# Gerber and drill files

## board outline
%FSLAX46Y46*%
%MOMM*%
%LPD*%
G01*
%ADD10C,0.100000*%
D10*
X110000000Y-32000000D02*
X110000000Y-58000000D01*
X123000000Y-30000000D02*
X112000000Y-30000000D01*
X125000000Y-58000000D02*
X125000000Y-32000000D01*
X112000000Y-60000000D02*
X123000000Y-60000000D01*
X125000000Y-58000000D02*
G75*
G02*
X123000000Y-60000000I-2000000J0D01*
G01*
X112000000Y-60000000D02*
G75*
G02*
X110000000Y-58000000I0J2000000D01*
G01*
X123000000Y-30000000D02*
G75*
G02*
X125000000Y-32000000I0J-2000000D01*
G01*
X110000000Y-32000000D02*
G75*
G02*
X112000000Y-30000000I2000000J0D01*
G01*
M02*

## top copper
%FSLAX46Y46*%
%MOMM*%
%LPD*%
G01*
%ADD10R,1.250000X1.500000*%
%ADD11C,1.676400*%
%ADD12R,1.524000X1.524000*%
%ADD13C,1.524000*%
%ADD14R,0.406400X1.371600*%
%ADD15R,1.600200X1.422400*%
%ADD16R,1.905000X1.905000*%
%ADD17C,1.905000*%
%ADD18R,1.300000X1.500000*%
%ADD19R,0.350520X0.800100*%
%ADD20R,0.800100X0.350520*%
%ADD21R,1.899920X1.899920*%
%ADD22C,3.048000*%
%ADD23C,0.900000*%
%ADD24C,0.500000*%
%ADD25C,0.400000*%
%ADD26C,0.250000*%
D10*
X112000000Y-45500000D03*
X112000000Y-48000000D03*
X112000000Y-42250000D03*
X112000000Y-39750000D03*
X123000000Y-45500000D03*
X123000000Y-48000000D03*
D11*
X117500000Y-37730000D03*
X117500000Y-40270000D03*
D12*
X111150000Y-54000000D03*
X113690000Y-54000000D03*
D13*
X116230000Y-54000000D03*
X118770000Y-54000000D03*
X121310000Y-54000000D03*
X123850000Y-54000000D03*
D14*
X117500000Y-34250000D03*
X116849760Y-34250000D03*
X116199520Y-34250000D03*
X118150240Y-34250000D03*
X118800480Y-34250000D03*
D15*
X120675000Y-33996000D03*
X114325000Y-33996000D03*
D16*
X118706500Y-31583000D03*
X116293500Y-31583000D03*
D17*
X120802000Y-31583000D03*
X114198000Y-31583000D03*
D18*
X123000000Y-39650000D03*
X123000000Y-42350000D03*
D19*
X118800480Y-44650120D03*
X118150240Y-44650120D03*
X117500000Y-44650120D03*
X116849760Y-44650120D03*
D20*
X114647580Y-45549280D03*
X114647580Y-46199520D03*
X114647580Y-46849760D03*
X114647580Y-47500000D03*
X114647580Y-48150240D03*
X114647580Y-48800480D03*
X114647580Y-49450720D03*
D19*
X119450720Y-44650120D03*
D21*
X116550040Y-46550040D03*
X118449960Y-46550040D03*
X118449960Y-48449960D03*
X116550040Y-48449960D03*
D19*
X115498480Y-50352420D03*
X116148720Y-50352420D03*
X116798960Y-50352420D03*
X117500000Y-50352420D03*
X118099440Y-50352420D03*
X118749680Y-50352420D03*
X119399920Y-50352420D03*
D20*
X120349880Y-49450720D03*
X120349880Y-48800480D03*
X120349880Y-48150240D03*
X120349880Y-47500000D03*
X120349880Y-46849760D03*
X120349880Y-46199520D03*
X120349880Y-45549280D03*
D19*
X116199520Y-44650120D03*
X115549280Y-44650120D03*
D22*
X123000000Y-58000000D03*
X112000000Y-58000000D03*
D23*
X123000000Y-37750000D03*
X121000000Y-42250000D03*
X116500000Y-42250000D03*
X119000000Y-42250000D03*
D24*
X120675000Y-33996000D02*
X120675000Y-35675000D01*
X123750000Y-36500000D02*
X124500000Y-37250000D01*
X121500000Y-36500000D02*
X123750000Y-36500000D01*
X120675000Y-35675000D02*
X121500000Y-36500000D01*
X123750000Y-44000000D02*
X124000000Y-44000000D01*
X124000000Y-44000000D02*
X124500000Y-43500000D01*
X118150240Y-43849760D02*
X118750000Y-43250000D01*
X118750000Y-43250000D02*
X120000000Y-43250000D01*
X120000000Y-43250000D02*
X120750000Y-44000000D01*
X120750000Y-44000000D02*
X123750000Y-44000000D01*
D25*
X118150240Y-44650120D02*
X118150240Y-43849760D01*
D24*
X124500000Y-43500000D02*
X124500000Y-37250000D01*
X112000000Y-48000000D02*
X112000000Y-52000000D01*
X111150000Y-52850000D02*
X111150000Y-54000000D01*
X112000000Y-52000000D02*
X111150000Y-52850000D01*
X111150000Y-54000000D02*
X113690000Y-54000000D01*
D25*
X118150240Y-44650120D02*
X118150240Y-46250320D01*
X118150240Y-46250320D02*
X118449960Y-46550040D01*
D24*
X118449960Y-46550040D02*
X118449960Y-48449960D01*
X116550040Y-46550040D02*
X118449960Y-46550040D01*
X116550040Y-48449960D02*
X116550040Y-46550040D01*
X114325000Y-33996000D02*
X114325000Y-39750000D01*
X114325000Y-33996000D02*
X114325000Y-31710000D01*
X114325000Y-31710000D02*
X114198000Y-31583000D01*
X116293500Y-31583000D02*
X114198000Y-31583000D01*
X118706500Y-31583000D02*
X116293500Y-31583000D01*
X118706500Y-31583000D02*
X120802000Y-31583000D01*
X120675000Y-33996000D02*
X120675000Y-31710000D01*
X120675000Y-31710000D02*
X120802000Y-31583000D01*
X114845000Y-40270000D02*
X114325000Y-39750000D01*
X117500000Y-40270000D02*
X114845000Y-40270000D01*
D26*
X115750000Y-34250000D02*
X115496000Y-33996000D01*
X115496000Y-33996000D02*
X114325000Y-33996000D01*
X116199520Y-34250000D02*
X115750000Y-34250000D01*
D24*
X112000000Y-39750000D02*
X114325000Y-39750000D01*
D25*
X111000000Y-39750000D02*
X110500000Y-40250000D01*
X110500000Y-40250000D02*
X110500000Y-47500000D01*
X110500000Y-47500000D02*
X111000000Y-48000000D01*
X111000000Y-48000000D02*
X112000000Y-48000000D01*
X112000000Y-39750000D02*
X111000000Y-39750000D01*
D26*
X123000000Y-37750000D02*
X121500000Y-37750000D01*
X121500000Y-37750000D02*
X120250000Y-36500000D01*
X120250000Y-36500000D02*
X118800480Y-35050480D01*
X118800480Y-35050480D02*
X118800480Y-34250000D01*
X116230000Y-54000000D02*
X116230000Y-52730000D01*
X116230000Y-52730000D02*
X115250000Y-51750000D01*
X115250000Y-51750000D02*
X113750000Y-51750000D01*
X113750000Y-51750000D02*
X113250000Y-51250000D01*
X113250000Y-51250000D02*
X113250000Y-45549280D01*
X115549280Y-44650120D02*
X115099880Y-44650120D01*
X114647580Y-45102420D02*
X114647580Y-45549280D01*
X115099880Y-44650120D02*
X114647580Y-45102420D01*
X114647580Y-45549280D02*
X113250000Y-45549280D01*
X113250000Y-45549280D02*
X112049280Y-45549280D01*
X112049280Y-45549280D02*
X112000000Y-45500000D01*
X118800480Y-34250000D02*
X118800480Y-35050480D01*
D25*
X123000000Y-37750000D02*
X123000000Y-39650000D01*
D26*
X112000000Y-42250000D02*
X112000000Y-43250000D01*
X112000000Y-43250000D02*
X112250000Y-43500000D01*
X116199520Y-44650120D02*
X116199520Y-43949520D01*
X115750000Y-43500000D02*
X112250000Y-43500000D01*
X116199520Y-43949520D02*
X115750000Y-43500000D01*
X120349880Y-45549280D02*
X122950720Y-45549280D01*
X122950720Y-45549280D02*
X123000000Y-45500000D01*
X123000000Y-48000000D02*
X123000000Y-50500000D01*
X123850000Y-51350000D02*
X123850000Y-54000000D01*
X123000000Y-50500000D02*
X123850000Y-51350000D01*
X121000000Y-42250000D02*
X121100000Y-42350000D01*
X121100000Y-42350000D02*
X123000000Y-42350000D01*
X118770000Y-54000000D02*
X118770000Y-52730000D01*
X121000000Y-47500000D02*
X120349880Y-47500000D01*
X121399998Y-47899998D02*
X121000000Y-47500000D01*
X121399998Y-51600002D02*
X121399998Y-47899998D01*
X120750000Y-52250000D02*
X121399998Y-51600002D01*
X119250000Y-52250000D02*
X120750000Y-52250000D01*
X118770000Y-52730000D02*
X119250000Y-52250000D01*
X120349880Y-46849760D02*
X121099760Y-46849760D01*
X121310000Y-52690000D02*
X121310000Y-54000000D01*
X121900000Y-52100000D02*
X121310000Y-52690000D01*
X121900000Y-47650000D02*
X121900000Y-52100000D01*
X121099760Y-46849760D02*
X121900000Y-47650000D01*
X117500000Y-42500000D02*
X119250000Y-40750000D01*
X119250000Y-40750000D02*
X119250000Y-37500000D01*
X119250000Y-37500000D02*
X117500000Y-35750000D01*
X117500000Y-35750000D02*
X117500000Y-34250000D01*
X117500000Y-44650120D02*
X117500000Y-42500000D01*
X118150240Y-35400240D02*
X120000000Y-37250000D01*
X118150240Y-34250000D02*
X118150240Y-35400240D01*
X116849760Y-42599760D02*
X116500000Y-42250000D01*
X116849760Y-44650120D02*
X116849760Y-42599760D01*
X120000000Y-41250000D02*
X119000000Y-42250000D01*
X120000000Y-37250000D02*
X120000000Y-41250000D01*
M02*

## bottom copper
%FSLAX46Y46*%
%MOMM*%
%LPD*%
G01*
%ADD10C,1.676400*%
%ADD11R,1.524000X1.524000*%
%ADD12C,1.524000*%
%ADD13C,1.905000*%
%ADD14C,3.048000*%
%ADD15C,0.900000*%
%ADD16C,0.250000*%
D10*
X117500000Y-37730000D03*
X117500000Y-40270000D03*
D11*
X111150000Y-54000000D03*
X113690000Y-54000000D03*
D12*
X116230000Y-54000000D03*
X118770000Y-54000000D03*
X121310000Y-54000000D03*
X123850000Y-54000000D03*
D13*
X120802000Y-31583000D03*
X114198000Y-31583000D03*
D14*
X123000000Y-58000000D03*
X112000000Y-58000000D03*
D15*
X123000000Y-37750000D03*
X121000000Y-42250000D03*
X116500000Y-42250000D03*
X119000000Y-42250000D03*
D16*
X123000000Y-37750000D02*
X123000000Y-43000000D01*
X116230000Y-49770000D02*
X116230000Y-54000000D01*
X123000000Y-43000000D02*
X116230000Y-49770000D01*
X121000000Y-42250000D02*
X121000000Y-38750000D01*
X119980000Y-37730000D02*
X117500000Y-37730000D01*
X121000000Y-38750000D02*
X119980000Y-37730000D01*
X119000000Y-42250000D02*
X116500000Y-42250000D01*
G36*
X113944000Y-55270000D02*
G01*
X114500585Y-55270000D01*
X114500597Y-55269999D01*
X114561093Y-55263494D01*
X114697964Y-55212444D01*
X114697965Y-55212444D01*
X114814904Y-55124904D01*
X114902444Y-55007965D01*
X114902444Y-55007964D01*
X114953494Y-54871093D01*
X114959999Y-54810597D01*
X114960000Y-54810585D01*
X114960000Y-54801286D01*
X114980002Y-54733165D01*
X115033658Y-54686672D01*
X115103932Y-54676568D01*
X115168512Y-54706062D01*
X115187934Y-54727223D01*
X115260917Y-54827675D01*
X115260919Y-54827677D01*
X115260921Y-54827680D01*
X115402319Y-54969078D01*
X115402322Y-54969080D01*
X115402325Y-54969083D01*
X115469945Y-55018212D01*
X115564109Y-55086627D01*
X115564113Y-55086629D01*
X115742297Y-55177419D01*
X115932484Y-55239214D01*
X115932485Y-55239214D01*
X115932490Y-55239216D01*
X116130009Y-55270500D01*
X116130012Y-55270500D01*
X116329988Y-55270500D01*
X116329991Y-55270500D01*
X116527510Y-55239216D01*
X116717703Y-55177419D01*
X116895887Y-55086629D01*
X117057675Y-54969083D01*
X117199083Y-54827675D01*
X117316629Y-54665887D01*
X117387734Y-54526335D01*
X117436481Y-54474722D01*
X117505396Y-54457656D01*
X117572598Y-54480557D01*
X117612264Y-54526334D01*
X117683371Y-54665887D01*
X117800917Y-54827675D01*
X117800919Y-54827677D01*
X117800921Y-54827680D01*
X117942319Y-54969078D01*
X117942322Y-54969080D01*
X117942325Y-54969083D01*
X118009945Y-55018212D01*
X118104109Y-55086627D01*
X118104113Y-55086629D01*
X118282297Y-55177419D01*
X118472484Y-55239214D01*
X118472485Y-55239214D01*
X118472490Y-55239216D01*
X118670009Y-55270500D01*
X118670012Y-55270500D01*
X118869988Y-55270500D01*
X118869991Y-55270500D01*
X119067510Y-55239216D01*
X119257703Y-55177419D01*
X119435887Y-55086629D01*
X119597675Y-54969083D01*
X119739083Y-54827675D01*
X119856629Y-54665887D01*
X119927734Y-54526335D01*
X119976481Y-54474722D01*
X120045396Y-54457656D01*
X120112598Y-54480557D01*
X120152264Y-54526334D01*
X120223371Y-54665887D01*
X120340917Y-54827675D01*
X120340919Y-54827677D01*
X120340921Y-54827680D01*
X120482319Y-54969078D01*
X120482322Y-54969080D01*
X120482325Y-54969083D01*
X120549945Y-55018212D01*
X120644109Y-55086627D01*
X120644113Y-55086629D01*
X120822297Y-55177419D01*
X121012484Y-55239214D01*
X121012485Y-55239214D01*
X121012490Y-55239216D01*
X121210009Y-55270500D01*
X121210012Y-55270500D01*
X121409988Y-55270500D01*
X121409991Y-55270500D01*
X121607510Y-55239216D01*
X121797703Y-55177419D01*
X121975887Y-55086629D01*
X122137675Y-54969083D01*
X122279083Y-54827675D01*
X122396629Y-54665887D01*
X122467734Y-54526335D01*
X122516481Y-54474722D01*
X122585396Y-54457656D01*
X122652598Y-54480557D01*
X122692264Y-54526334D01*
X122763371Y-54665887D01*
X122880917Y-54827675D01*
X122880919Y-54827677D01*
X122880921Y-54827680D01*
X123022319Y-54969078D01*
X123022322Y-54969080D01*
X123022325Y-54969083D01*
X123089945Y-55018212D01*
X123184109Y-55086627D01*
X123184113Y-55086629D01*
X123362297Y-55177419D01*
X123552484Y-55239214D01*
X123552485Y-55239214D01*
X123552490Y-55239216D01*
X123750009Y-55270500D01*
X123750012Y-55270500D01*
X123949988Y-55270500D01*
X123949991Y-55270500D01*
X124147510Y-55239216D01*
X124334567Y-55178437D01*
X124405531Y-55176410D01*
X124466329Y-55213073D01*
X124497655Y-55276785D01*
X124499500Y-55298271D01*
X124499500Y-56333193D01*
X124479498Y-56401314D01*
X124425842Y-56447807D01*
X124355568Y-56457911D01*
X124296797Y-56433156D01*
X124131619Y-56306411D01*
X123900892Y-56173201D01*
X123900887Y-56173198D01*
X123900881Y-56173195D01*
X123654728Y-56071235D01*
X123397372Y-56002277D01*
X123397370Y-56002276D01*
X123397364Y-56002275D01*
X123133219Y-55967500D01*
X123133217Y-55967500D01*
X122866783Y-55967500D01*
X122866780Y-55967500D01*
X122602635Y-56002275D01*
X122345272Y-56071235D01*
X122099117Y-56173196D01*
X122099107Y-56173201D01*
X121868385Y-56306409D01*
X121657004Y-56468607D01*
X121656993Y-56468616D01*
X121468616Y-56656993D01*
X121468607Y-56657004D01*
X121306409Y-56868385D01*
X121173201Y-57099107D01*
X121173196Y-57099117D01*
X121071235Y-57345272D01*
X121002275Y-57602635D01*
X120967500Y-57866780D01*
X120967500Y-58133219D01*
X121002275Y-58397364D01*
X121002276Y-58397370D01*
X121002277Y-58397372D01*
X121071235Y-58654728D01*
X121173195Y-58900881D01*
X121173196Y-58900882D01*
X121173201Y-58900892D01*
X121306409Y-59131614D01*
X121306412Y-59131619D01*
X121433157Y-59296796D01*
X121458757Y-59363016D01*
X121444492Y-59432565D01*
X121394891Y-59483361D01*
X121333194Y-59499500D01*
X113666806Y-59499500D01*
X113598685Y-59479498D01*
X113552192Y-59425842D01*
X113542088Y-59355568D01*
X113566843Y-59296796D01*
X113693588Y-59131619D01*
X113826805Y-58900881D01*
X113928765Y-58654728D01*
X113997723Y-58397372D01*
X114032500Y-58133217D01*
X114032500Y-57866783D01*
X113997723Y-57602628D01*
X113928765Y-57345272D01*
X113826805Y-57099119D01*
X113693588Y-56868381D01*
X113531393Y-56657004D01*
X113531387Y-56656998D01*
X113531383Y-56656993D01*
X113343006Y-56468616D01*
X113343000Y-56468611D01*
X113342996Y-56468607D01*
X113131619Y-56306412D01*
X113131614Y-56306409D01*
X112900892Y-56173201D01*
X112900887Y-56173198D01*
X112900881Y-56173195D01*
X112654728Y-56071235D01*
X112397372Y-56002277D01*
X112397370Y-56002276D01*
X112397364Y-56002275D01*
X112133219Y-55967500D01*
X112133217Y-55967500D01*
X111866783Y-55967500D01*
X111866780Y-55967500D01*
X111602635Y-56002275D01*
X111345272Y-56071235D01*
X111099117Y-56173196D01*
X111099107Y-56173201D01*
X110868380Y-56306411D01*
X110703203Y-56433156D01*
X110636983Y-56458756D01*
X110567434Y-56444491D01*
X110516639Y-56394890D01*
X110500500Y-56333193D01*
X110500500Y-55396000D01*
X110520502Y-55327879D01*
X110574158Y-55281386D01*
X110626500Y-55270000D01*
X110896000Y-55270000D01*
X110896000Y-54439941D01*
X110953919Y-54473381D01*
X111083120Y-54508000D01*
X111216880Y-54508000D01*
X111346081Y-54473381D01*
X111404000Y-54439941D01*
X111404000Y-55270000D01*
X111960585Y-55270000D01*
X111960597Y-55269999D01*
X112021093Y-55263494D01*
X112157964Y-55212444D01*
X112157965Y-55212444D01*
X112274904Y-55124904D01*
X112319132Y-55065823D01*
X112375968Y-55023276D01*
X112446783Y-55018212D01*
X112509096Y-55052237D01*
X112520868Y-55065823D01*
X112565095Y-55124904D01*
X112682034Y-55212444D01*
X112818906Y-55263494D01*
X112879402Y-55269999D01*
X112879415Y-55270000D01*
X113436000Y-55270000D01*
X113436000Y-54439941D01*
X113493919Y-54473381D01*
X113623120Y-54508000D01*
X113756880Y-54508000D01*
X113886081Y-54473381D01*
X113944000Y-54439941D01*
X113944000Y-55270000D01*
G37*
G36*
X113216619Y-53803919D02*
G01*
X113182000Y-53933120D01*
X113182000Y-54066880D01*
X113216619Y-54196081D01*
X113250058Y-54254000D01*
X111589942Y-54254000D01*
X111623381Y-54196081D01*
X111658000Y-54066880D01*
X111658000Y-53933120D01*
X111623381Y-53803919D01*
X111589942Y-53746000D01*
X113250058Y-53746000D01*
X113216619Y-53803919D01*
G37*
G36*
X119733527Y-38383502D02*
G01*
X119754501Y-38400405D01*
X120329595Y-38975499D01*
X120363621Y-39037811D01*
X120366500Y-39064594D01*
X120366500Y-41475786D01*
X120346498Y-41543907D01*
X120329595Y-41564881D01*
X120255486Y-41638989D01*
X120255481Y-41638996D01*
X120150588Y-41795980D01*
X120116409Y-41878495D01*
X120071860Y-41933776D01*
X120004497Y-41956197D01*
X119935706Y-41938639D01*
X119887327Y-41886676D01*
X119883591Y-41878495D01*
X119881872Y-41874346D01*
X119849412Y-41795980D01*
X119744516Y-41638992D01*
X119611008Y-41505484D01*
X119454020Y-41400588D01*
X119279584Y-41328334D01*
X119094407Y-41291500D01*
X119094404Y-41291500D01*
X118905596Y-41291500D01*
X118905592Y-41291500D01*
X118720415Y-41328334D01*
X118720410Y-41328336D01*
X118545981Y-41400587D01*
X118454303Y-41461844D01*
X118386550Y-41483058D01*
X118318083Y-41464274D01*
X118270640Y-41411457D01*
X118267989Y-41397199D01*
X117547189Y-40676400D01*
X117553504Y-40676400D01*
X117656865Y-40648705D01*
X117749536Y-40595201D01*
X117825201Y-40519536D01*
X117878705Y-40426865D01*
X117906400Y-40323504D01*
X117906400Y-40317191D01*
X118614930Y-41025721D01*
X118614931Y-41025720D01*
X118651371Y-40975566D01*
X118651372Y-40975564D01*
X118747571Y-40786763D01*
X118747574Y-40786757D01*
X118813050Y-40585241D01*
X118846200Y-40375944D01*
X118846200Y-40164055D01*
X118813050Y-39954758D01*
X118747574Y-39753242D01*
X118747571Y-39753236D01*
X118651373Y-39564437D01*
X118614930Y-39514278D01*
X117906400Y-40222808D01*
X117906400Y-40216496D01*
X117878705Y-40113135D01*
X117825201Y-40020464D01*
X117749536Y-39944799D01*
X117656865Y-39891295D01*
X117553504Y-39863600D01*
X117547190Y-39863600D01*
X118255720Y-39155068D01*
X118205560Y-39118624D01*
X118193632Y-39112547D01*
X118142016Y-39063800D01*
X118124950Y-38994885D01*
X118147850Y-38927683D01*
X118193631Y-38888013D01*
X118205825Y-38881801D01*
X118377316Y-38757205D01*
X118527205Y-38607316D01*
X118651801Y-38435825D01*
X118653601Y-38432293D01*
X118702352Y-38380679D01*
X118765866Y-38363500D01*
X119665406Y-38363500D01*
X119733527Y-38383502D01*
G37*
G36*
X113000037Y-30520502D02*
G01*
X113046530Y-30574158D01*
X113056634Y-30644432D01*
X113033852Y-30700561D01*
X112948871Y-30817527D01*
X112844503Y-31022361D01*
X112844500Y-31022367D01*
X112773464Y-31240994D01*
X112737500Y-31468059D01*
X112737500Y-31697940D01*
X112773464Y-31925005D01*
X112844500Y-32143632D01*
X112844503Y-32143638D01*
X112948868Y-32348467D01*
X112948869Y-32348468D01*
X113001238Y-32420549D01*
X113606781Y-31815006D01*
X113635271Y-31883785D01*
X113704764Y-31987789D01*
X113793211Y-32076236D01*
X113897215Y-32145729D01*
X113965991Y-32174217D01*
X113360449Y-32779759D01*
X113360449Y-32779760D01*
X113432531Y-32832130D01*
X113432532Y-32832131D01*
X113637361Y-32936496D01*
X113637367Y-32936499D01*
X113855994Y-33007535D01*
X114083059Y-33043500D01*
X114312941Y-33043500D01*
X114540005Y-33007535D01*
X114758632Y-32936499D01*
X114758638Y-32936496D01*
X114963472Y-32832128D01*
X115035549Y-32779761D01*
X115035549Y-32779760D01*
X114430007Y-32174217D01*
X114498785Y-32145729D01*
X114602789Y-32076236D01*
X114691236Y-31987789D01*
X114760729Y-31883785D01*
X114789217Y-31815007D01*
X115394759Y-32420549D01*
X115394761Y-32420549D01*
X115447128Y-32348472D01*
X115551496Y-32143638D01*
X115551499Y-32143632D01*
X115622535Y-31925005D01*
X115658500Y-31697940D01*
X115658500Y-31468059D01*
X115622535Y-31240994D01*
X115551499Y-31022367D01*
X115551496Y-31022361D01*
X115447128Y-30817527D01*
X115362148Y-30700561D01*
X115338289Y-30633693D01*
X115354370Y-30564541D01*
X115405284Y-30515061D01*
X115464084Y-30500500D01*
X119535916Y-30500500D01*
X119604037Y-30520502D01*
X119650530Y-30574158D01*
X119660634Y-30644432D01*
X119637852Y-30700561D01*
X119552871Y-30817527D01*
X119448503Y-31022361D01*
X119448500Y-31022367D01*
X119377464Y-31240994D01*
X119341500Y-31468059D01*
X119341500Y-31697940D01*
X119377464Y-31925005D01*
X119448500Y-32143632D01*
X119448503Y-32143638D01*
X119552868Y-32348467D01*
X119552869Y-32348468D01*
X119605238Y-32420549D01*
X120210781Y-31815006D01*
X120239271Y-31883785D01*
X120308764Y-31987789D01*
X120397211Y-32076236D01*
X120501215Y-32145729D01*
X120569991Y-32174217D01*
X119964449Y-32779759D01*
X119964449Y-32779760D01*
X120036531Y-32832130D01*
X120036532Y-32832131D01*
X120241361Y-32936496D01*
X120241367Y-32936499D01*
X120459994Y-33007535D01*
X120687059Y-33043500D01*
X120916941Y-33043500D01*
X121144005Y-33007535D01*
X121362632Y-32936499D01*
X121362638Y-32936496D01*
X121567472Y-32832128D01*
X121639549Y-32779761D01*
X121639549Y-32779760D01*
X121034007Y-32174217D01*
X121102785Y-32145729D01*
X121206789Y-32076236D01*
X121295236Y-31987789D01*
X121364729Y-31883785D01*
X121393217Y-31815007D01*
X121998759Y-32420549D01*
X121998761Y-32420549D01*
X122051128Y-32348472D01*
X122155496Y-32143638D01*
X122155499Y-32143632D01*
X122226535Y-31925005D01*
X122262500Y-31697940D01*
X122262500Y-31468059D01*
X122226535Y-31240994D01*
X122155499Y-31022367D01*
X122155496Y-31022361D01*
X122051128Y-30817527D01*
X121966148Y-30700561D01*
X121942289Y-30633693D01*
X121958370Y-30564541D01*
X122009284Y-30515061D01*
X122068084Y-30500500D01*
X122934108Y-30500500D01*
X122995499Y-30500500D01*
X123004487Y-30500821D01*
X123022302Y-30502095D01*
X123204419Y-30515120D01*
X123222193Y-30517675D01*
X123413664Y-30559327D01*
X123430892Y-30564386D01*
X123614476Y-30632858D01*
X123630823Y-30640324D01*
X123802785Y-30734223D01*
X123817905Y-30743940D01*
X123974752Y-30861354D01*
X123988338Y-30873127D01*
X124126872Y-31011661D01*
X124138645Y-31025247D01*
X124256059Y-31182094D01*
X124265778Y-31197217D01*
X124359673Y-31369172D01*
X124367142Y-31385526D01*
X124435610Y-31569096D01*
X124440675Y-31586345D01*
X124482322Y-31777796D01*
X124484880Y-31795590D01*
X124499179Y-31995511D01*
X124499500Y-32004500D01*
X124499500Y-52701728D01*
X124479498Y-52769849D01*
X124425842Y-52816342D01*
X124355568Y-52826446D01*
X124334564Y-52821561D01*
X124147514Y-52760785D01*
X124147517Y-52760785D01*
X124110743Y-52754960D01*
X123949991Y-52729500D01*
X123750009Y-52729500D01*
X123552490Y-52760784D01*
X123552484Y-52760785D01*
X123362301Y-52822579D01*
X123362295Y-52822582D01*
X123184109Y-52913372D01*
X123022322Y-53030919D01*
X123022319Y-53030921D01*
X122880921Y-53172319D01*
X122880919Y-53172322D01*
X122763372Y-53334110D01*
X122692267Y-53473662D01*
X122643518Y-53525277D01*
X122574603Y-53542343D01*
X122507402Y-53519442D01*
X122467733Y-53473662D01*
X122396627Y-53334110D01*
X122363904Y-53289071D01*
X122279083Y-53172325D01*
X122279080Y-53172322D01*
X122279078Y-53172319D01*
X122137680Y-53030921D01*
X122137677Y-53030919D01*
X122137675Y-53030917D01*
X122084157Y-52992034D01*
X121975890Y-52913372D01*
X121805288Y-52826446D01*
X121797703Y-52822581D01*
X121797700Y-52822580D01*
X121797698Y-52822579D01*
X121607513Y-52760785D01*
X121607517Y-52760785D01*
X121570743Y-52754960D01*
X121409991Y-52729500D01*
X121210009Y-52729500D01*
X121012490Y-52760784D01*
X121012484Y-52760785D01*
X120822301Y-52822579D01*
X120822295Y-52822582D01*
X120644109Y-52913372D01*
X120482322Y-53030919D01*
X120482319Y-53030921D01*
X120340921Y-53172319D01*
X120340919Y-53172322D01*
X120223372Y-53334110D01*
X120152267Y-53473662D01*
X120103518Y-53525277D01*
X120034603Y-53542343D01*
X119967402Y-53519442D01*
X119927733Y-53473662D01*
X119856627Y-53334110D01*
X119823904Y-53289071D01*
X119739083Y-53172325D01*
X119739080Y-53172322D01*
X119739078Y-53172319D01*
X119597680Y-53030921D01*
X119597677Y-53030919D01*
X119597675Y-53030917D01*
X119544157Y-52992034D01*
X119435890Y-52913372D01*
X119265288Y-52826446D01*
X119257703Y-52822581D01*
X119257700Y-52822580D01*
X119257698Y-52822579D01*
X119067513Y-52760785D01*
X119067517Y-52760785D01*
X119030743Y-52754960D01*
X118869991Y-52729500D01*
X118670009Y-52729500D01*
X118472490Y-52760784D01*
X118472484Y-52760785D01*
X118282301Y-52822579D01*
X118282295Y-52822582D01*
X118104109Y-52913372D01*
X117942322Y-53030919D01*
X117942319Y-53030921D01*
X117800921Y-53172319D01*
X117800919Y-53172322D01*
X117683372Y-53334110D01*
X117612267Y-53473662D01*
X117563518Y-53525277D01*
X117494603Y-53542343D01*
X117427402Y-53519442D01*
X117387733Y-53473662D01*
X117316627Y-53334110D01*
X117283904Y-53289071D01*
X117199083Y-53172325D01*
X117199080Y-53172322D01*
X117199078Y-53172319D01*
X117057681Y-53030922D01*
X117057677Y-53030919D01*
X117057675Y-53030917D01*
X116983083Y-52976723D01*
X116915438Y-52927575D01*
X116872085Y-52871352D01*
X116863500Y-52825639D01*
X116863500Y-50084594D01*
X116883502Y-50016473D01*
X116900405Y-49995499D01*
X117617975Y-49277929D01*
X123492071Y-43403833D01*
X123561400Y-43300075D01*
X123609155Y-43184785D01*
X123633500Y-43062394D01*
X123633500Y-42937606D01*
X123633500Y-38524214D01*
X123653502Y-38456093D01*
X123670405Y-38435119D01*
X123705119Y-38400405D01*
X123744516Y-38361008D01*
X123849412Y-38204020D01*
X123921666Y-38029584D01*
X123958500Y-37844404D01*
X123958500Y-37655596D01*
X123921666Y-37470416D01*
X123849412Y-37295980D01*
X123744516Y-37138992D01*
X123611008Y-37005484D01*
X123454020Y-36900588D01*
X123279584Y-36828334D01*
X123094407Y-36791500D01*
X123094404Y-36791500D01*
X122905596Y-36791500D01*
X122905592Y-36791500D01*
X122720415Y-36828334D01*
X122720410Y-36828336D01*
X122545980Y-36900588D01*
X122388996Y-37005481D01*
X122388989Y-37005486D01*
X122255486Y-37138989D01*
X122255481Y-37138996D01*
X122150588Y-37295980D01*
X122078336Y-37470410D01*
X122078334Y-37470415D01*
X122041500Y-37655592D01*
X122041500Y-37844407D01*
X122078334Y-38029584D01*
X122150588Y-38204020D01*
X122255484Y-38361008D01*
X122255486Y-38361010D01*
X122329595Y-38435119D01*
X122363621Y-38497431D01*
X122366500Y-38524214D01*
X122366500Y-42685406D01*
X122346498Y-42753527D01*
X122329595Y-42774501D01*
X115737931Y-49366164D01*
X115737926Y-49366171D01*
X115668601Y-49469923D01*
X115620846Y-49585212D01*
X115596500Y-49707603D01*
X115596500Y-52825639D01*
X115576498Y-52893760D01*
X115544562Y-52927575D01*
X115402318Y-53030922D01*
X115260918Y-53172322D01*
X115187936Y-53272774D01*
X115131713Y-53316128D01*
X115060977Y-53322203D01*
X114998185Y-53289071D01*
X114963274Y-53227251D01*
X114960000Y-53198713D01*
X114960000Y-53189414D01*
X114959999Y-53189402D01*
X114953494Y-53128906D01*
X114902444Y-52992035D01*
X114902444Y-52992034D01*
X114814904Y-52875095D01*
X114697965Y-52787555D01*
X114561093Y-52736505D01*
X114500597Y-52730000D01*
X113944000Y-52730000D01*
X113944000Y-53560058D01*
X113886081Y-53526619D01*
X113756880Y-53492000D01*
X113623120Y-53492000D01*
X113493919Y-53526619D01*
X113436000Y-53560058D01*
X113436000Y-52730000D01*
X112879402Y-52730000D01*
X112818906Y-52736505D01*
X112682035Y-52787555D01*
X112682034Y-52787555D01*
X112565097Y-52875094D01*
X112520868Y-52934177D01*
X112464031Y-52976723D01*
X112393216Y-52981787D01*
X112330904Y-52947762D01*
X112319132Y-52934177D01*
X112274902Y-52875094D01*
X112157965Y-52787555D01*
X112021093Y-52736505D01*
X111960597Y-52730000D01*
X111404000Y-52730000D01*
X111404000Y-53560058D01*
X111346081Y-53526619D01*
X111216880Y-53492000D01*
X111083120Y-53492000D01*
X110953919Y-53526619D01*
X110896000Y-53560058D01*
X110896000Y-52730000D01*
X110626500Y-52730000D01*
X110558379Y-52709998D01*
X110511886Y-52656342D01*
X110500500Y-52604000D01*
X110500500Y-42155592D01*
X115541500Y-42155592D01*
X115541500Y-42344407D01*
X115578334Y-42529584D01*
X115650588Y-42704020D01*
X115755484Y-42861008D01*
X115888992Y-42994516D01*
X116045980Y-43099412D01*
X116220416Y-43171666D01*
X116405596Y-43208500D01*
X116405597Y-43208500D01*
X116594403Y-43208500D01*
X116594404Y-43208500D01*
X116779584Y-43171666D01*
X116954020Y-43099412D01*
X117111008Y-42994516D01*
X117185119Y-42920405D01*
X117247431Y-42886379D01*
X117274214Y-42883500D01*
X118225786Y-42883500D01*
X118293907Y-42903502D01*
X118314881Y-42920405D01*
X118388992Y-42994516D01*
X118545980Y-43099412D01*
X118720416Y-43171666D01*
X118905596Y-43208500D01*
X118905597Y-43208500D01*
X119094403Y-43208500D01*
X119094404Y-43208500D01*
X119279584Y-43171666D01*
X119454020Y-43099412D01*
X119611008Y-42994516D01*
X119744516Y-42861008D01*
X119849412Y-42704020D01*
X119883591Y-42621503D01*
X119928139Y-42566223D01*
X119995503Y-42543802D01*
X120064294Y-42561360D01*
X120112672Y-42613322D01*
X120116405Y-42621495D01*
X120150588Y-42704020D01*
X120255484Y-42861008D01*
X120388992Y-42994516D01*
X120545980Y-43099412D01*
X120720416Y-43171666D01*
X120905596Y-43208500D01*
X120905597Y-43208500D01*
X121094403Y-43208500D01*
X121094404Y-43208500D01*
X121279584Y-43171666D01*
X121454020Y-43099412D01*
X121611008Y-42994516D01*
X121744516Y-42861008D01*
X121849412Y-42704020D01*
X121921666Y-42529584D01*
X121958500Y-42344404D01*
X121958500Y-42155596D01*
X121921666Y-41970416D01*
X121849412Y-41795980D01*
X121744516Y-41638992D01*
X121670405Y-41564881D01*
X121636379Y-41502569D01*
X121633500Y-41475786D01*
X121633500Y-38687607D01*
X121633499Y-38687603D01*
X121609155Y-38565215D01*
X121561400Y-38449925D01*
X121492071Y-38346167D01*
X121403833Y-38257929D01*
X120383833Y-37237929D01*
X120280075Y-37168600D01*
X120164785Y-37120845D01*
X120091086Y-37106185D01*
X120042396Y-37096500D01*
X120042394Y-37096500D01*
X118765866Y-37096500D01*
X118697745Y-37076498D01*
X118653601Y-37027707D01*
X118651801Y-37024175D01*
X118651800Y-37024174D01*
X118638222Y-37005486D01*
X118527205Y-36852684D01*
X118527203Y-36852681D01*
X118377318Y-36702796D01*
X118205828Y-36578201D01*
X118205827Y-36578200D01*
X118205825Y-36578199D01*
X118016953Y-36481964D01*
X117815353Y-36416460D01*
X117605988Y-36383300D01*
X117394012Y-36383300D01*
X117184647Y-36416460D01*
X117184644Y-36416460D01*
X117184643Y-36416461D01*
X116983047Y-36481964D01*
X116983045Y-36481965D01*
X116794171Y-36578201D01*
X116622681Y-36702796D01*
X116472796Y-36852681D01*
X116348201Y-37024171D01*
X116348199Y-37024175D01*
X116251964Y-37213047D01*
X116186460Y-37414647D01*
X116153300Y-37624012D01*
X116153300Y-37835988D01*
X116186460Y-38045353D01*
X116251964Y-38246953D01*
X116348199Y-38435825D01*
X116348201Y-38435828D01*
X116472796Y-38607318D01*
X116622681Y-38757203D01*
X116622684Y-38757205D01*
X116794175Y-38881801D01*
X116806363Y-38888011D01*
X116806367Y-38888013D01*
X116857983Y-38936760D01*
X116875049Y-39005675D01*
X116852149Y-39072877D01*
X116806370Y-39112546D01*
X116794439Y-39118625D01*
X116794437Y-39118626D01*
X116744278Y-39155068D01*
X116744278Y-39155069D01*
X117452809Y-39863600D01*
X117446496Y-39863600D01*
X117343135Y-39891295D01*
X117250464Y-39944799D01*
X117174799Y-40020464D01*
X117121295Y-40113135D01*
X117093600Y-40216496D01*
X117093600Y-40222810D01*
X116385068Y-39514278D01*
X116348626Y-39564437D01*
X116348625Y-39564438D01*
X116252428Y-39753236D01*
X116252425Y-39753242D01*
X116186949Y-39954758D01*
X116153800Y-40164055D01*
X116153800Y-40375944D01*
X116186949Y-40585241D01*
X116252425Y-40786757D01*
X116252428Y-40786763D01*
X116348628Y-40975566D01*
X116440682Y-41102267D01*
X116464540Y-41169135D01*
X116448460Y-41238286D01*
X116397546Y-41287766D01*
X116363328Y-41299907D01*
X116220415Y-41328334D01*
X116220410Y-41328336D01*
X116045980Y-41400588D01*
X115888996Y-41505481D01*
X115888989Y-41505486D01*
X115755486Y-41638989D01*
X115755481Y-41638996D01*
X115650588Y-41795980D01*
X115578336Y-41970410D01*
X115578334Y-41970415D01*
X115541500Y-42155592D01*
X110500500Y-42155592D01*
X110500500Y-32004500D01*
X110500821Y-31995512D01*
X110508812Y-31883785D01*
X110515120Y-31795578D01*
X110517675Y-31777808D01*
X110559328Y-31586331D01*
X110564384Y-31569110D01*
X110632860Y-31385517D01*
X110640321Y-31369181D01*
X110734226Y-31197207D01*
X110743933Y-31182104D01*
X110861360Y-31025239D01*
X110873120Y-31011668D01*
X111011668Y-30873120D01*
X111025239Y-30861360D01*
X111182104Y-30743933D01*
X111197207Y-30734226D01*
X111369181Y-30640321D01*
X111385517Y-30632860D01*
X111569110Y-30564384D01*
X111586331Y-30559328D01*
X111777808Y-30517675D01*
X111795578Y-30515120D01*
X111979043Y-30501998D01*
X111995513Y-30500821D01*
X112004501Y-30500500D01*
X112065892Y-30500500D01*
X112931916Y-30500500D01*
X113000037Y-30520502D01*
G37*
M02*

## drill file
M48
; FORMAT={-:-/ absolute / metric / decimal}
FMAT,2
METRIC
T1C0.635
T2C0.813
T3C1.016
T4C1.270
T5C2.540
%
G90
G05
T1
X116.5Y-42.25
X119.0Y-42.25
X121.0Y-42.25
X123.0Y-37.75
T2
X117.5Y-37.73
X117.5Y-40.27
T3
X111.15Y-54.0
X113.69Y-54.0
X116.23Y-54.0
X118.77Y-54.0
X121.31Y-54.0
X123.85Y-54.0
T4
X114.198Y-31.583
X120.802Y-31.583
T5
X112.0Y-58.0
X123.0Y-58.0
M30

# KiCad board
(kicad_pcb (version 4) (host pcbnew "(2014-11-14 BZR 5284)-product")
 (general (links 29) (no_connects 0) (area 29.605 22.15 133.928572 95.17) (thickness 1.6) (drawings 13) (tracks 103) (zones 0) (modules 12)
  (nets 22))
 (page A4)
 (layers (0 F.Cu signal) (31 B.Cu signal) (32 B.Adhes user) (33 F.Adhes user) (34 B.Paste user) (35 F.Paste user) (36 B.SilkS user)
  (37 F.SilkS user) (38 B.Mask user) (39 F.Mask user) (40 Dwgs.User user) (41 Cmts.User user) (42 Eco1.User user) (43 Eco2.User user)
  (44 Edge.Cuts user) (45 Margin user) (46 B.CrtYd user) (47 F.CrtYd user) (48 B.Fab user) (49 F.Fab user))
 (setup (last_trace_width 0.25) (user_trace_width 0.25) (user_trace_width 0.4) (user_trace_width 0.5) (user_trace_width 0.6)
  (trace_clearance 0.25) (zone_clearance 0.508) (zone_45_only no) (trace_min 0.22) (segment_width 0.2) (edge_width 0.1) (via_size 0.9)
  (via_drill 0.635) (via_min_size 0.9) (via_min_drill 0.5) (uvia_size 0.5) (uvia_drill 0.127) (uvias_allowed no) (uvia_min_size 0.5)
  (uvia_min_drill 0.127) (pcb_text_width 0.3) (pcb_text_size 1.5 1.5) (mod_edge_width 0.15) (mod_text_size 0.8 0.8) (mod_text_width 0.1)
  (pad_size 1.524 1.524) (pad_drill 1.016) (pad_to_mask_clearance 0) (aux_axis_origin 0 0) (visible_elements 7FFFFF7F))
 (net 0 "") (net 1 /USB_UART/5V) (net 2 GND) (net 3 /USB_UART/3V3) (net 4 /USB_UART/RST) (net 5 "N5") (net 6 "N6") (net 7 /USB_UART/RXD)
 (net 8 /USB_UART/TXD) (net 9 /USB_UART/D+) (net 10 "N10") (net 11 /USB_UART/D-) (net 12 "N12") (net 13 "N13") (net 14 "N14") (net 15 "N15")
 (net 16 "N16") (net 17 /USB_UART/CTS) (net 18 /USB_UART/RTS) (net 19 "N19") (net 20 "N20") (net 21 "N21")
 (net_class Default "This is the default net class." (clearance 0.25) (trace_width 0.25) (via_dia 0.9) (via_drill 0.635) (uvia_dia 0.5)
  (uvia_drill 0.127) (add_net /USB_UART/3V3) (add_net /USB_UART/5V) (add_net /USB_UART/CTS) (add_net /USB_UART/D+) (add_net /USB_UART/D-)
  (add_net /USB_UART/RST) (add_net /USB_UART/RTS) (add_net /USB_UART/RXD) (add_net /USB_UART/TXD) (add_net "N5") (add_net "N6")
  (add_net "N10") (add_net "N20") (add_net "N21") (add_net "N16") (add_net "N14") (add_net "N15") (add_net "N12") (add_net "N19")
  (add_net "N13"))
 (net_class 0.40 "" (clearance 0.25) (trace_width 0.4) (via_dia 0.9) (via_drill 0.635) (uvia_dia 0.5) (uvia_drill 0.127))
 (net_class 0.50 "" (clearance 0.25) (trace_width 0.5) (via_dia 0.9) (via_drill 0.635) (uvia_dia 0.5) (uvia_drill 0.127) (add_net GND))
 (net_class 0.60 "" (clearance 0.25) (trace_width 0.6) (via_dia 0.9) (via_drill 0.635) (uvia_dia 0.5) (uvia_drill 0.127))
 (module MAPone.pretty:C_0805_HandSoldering (layer F.Cu) (at 112 46.75 270)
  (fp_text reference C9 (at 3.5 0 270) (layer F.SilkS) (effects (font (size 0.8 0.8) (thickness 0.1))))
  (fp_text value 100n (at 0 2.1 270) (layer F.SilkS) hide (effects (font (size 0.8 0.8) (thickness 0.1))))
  (pad 1 smd rect (at -1.25 0 270) (size 1.5 1.25) (layers F.Cu F.Paste F.Mask) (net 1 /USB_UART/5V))
  (pad 2 smd rect (at 1.25 0 270) (size 1.5 1.25) (layers F.Cu F.Paste F.Mask) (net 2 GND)))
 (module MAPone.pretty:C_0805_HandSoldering (layer F.Cu) (at 112 41 90)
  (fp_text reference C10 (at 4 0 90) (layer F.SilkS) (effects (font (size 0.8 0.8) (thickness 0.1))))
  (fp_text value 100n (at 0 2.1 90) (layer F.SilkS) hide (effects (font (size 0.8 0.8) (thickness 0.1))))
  (pad 1 smd rect (at -1.25 0 90) (size 1.5 1.25) (layers F.Cu F.Paste F.Mask) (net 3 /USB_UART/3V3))
  (pad 2 smd rect (at 1.25 0 90) (size 1.5 1.25) (layers F.Cu F.Paste F.Mask) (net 2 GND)))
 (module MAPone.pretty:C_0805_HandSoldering (layer F.Cu) (at 123 46.75 270)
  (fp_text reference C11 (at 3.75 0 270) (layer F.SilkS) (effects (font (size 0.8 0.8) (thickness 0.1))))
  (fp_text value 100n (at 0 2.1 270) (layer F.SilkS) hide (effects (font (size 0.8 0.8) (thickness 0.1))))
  (pad 1 smd rect (at -1.25 0 270) (size 1.5 1.25) (layers F.Cu F.Paste F.Mask) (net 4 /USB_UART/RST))
  (pad 2 smd rect (at 1.25 0 270) (size 1.5 1.25) (layers F.Cu F.Paste F.Mask) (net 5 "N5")))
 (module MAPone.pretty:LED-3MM (layer F.Cu) (at 117.5 39 270)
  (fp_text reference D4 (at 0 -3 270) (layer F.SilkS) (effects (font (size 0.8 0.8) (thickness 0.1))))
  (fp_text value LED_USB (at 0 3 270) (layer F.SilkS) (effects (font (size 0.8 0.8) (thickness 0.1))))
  (pad 1 thru_hole circle (at -1.27 0 270) (size 1.6764 1.6764) (drill 0.8128) (layers *.Cu *.Mask F.SilkS) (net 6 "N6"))
  (pad 2 thru_hole circle (at 1.27 0 270) (size 1.6764 1.6764) (drill 0.8128) (layers *.Cu *.Mask F.SilkS) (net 2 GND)))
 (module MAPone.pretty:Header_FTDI (layer F.Cu) (at 117.5 54)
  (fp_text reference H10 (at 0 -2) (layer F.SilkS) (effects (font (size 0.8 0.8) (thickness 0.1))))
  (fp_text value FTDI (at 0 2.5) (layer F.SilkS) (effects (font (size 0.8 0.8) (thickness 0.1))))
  (pad 1 thru_hole rect (at -6.35 0) (size 1.524 1.524) (drill 1.016) (layers *.Cu *.Mask F.SilkS) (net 2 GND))
  (pad 2 thru_hole rect (at -3.81 0) (size 1.524 1.524) (drill 1.016) (layers *.Cu *.Mask F.SilkS) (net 2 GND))
  (pad 3 thru_hole circle (at -1.27 0) (size 1.524 1.524) (drill 1.016) (layers *.Cu *.Mask F.SilkS) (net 1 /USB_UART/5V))
  (pad 4 thru_hole circle (at 1.27 0) (size 1.524 1.524) (drill 1.016) (layers *.Cu *.Mask F.SilkS) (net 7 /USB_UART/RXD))
  (pad 5 thru_hole circle (at 3.81 0) (size 1.524 1.524) (drill 1.016) (layers *.Cu *.Mask F.SilkS) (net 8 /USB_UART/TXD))
  (pad 6 thru_hole circle (at 6.35 0) (size 1.524 1.524) (drill 1.016) (layers *.Cu *.Mask F.SilkS) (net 5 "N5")))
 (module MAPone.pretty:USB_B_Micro (layer F.Cu) (at 117.5 34.25 270)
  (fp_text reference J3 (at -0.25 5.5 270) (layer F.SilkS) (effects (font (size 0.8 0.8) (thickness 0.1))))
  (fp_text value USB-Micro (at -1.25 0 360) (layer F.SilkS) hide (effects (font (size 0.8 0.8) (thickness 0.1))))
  (pad 3 smd rect (at 0 0 270) (size 1.3716 0.4064) (layers F.Cu F.Paste F.Mask) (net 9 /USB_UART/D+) (clearance 0.2032))
  (pad 4 smd rect (at 0 0.65024 270) (size 1.3716 0.4064) (layers F.Cu F.Paste F.Mask) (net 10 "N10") (clearance 0.2032))
  (pad 5 smd rect (at 0 1.30048 270) (size 1.3716 0.4064) (layers F.Cu F.Paste F.Mask) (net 2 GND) (clearance 0.2032))
  (pad 2 smd rect (at 0 -0.65024 270) (size 1.3716 0.4064) (layers F.Cu F.Paste F.Mask) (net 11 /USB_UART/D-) (clearance 0.2032))
  (pad 1 smd rect (at 0 -1.30048 270) (size 1.3716 0.4064) (layers F.Cu F.Paste F.Mask) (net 1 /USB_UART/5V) (clearance 0.2032))
  (pad T1 smd rect (at -0.254 -3.175 270) (size 1.4224 1.6002) (layers F.Cu F.Paste F.Mask) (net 2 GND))
  (pad T2 smd rect (at -0.254 3.175 270) (size 1.4224 1.6002) (layers F.Cu F.Paste F.Mask) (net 2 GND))
  (pad T3 smd rect (at -2.667 -1.2065 270) (size 1.905 1.905) (layers F.Cu F.Paste F.Mask) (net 2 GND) (clearance 0.2032))
  (pad T4 smd rect (at -2.667 1.2065 270) (size 1.905 1.905) (layers F.Cu F.Paste F.Mask) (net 2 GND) (clearance 0.2032))
  (pad T5 thru_hole circle (at -2.667 -3.302 270) (size 1.905 1.905) (drill 1.27) (layers *.Cu *.Paste *.Mask F.SilkS) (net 2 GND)
   (clearance 0.2032))
  (pad T6 thru_hole circle (at -2.667 3.302 270) (size 1.905 1.905) (drill 1.27) (layers *.Cu *.Paste *.Mask F.SilkS) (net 2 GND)
   (clearance 0.2032)))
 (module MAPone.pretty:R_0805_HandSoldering (layer F.Cu) (at 123 41 270)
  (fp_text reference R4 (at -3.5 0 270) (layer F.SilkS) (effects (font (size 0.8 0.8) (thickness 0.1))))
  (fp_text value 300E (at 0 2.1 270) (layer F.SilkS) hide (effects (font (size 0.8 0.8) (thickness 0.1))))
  (pad 1 smd rect (at -1.35 0 270) (size 1.5 1.3) (layers F.Cu F.Paste F.Mask) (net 1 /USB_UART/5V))
  (pad 2 smd rect (at 1.35 0 270) (size 1.5 1.3) (layers F.Cu F.Paste F.Mask) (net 6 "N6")))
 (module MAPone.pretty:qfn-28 (layer F.Cu) (at 117.5 47.5 180)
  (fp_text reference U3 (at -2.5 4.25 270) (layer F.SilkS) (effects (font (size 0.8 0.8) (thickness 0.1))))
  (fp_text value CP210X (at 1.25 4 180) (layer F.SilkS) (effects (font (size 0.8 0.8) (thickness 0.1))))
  (pad 2 smd rect (at -1.30048 2.84988 180) (size 0.35052 0.8001) (layers F.Cu F.Paste F.Mask) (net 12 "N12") (solder_mask_margin 0.07112)
   (clearance 0.1))
  (pad 3 smd rect (at -0.65024 2.84988 180) (size 0.35052 0.8001) (layers F.Cu F.Paste F.Mask) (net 2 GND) (solder_mask_margin 0.07112)
   (clearance 0.1))
  (pad 4 smd rect (at 0 2.84988 180) (size 0.35052 0.8001) (layers F.Cu F.Paste F.Mask) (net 9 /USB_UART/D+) (solder_mask_margin 0.07112)
   (clearance 0.1))
  (pad 5 smd rect (at 0.65024 2.84988 180) (size 0.35052 0.8001) (layers F.Cu F.Paste F.Mask) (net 11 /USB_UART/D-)
   (solder_mask_margin 0.07112) (clearance 0.1))
  (pad 8 smd rect (at 2.85242 1.95072 180) (size 0.8001 0.35052) (layers F.Cu F.Paste F.Mask) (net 1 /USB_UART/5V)
   (solder_mask_margin 0.07112) (clearance 0.1))
  (pad 9 smd rect (at 2.85242 1.30048 180) (size 0.8001 0.35052) (layers F.Cu F.Paste F.Mask) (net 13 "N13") (solder_mask_margin 0.07112)
   (clearance 0.1))
  (pad 10 smd rect (at 2.85242 0.65024 180) (size 0.8001 0.35052) (layers F.Cu F.Paste F.Mask) (solder_mask_margin 0.07112) (clearance 0.1))
  (pad 11 smd rect (at 2.85242 0 180) (size 0.8001 0.35052) (layers F.Cu F.Paste F.Mask) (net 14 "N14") (solder_mask_margin 0.07112)
   (clearance 0.1))
  (pad 12 smd rect (at 2.85242 -0.65024 180) (size 0.8001 0.35052) (layers F.Cu F.Paste F.Mask) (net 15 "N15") (solder_mask_margin 0.07112)
   (clearance 0.1))
  (pad 13 smd rect (at 2.85242 -1.30048 180) (size 0.8001 0.35052) (layers F.Cu F.Paste F.Mask) (solder_mask_margin 0.07112) (clearance 0.1))
  (pad 14 smd rect (at 2.85242 -1.95072 180) (size 0.8001 0.35052) (layers F.Cu F.Paste F.Mask) (solder_mask_margin 0.07112) (clearance 0.1))
  (pad 1 smd rect (at -1.95072 2.84988 180) (size 0.35052 0.8001) (layers F.Cu F.Paste F.Mask) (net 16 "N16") (solder_mask_margin 0.07112)
   (clearance 0.1))
  (pad 29 smd rect (at 0.94996 0.94996 180) (size 1.89992 1.89992) (layers F.Cu F.Paste F.Mask) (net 2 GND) (solder_mask_margin 0.07112)
   (solder_paste_margin -0.09906))
  (pad 29 smd rect (at -0.94996 0.94996 180) (size 1.89992 1.89992) (layers F.Cu F.Paste F.Mask) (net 2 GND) (solder_mask_margin 0.07112)
   (solder_paste_margin -0.09906))
  (pad 29 smd rect (at -0.94996 -0.94996 180) (size 1.89992 1.89992) (layers F.Cu F.Paste F.Mask) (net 2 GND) (solder_mask_margin 0.07112)
   (solder_paste_margin -0.09906))
  (pad 29 smd rect (at 0.94996 -0.94996 180) (size 1.89992 1.89992) (layers F.Cu F.Paste F.Mask) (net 2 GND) (solder_mask_margin 0.07112)
   (solder_paste_margin -0.09906))
  (pad 15 smd rect (at 2.00152 -2.85242 180) (size 0.35052 0.8001) (layers F.Cu F.Paste F.Mask) (solder_mask_margin 0.07112) (clearance 0.1))
  (pad 16 smd rect (at 1.35128 -2.85242 180) (size 0.35052 0.8001) (layers F.Cu F.Paste F.Mask) (solder_mask_margin 0.07112) (clearance 0.1))
  (pad 17 smd rect (at 0.70104 -2.85242 180) (size 0.35052 0.8001) (layers F.Cu F.Paste F.Mask) (solder_mask_margin 0.07112) (clearance 0.1))
  (pad 18 smd rect (at 0 -2.85242 180) (size 0.35052 0.8001) (layers F.Cu F.Paste F.Mask) (solder_mask_margin 0.07112) (clearance 0.1))
  (pad 19 smd rect (at -0.59944 -2.85242 180) (size 0.35052 0.8001) (layers F.Cu F.Paste F.Mask) (solder_mask_margin 0.07112)
   (clearance 0.1))
  (pad 20 smd rect (at -1.24968 -2.85242 180) (size 0.35052 0.8001) (layers F.Cu F.Paste F.Mask) (solder_mask_margin 0.07112)
   (clearance 0.1))
  (pad 21 smd rect (at -1.89992 -2.85242 180) (size 0.35052 0.8001) (layers F.Cu F.Paste F.Mask) (solder_mask_margin 0.07112)
   (clearance 0.1))
  (pad 22 smd rect (at -2.84988 -1.95072 180) (size 0.8001 0.35052) (layers F.Cu F.Paste F.Mask) (solder_mask_margin 0.07112)
   (clearance 0.1))
  (pad 23 smd rect (at -2.84988 -1.30048 180) (size 0.8001 0.35052) (layers F.Cu F.Paste F.Mask) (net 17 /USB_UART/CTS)
   (solder_mask_margin 0.07112) (clearance 0.1))
  (pad 24 smd rect (at -2.84988 -0.65024 180) (size 0.8001 0.35052) (layers F.Cu F.Paste F.Mask) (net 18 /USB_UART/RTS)
   (solder_mask_margin 0.07112) (clearance 0.1))
  (pad 25 smd rect (at -2.84988 0 180) (size 0.8001 0.35052) (layers F.Cu F.Paste F.Mask) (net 7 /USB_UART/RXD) (solder_mask_margin 0.07112)
   (clearance 0.1))
  (pad 26 smd rect (at -2.84988 0.65024 180) (size 0.8001 0.35052) (layers F.Cu F.Paste F.Mask) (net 8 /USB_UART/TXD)
   (solder_mask_margin 0.07112) (clearance 0.1))
  (pad 27 smd rect (at -2.84988 1.30048 180) (size 0.8001 0.35052) (layers F.Cu F.Paste F.Mask) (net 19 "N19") (solder_mask_margin 0.07112)
   (clearance 0.1))
  (pad 28 smd rect (at -2.84988 1.95072 180) (size 0.8001 0.35052) (layers F.Cu F.Paste F.Mask) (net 4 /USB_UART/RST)
   (solder_mask_margin 0.07112) (clearance 0.1))
  (pad 6 smd rect (at 1.30048 2.84988 180) (size 0.35052 0.8001) (layers F.Cu F.Paste F.Mask) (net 3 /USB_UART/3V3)
   (solder_mask_margin 0.07112) (clearance 0.1))
  (pad 7 smd rect (at 1.95072 2.84988 180) (size 0.35052 0.8001) (layers F.Cu F.Paste F.Mask) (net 1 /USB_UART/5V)
   (solder_mask_margin 0.07112) (clearance 0.1)))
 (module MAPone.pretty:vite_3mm (layer F.Cu) (at 123 58)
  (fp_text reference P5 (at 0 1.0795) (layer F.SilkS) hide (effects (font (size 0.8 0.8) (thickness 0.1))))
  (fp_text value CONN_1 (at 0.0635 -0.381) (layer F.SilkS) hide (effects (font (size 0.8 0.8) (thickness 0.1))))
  (pad 1 thru_hole circle (at 0 0) (size 3.048 3.048) (drill 2.54) (layers *.Cu *.SilkS *.Mask) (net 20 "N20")))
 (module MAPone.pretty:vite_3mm (layer F.Cu) (at 112 58)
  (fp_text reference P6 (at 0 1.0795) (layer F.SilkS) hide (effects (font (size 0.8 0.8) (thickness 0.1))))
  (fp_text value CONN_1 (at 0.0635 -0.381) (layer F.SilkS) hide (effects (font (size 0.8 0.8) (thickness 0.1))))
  (pad 1 thru_hole circle (at 0 0) (size 3.048 3.048) (drill 2.54) (layers *.Cu *.SilkS *.Mask) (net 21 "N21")))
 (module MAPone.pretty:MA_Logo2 (layer B.Cu) (at 117.5 48 180)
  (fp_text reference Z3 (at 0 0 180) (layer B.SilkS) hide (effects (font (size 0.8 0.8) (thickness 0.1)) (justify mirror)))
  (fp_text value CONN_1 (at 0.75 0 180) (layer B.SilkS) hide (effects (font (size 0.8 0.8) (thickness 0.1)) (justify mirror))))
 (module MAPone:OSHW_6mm (layer B.Cu) (at 117.5 34.5 180)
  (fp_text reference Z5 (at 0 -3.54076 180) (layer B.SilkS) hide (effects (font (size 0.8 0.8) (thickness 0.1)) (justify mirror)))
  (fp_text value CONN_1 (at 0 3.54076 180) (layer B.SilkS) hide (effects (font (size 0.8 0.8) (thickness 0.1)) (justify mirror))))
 (gr_line (start 110 32) (end 110 58) (angle 90) (layer Edge.Cuts) (width 0.1))
 (gr_line (start 123 30) (end 112 30) (angle 90) (layer Edge.Cuts) (width 0.1))
 (gr_line (start 125 58) (end 125 32) (angle 90) (layer Edge.Cuts) (width 0.1))
 (gr_line (start 112 60) (end 123 60) (angle 90) (layer Edge.Cuts) (width 0.1))
 (gr_arc (start 123 58) (end 125 58) (angle 90) (layer Edge.Cuts) (width 0.1))
 (gr_arc (start 112 58) (end 112 60) (angle 90) (layer Edge.Cuts) (width 0.1))
 (gr_arc (start 123 32) (end 123 30) (angle 90) (layer Edge.Cuts) (width 0.1))
 (gr_arc (start 112 32) (end 110 32) (angle 90) (layer Edge.Cuts) (width 0.1))
 (segment (start 120.675 33.996) (end 120.675 35.675) (width 0.5) (layer F.Cu) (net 2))
 (segment (start 123.75 36.5) (end 124.5 37.25) (width 0.5) (layer F.Cu) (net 2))
 (segment (start 121.5 36.5) (end 123.75 36.5) (width 0.5) (layer F.Cu) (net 2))
 (segment (start 120.675 35.675) (end 121.5 36.5) (width 0.5) (layer F.Cu) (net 2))
 (segment (start 123.75 44) (end 124 44) (width 0.5) (layer F.Cu) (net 2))
 (segment (start 124 44) (end 124.5 43.5) (width 0.5) (layer F.Cu) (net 2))
 (segment (start 118.15024 43.84976) (end 118.75 43.25) (width 0.5) (layer F.Cu) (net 2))
 (segment (start 118.75 43.25) (end 120 43.25) (width 0.5) (layer F.Cu) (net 2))
 (segment (start 120 43.25) (end 120.75 44) (width 0.5) (layer F.Cu) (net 2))
 (segment (start 120.75 44) (end 123.75 44) (width 0.5) (layer F.Cu) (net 2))
 (segment (start 118.15024 44.65012) (end 118.15024 43.84976) (width 0.4) (layer F.Cu) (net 2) (status 10))
 (segment (start 124.5 43.5) (end 124.5 37.25) (width 0.5) (layer F.Cu) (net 2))
 (segment (start 112 48) (end 112 52) (width 0.5) (layer F.Cu) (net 2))
 (segment (start 111.15 52.85) (end 111.15 54) (width 0.5) (layer F.Cu) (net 2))
 (segment (start 112 52) (end 111.15 52.85) (width 0.5) (layer F.Cu) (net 2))
 (segment (start 111.15 54) (end 113.69 54) (width 0.5) (layer F.Cu) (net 2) (status 30))
 (segment (start 118.15024 44.65012) (end 118.15024 46.25032) (width 0.4) (layer F.Cu) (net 2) (status 30))
 (segment (start 118.15024 46.25032) (end 118.44996 46.55004) (width 0.4) (layer F.Cu) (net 2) (status 30))
 (segment (start 118.44996 46.55004) (end 118.44996 48.44996) (width 0.5) (layer F.Cu) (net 2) (status 30))
 (segment (start 116.55004 46.55004) (end 118.44996 46.55004) (width 0.5) (layer F.Cu) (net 2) (status 30))
 (segment (start 116.55004 48.44996) (end 116.55004 46.55004) (width 0.5) (layer F.Cu) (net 2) (status 30))
 (segment (start 114.325 33.996) (end 114.325 39.75) (width 0.5) (layer F.Cu) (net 2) (status 10))
 (segment (start 114.325 33.996) (end 114.325 31.71) (width 0.5) (layer F.Cu) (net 2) (status 30))
 (segment (start 114.325 31.71) (end 114.198 31.583) (width 0.5) (layer F.Cu) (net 2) (status 30))
 (segment (start 116.2935 31.583) (end 114.198 31.583) (width 0.5) (layer F.Cu) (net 2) (status 30))
 (segment (start 118.7065 31.583) (end 116.2935 31.583) (width 0.5) (layer F.Cu) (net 2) (status 30))
 (segment (start 118.7065 31.583) (end 120.802 31.583) (width 0.5) (layer F.Cu) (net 2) (status 30))
 (segment (start 120.675 33.996) (end 120.675 31.71) (width 0.5) (layer F.Cu) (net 2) (status 30))
 (segment (start 120.675 31.71) (end 120.802 31.583) (width 0.5) (layer F.Cu) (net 2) (status 30))
 (segment (start 114.845 40.27) (end 114.325 39.75) (width 0.5) (layer F.Cu) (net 2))
 (segment (start 117.5 40.27) (end 114.845 40.27) (width 0.5) (layer F.Cu) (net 2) (status 10))
 (segment (start 115.75 34.25) (end 115.496 33.996) (width 0.25) (layer F.Cu) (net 2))
 (segment (start 115.496 33.996) (end 114.325 33.996) (width 0.25) (layer F.Cu) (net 2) (status 20))
 (segment (start 116.19952 34.25) (end 115.75 34.25) (width 0.25) (layer F.Cu) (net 2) (status 10))
 (segment (start 112 39.75) (end 114.325 39.75) (width 0.5) (layer F.Cu) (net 2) (status 10))
 (segment (start 111 39.75) (end 110.5 40.25) (width 0.4) (layer F.Cu) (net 2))
 (segment (start 110.5 40.25) (end 110.5 47.5) (width 0.4) (layer F.Cu) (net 2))
 (segment (start 110.5 47.5) (end 111 48) (width 0.4) (layer F.Cu) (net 2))
 (segment (start 111 48) (end 112 48) (width 0.4) (layer F.Cu) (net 2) (status 20))
 (segment (start 112 39.75) (end 111 39.75) (width 0.4) (layer F.Cu) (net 2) (status 10))
 (segment (start 123 37.75) (end 121.5 37.75) (width 0.25) (layer F.Cu) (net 1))
 (segment (start 121.5 37.75) (end 120.25 36.5) (width 0.25) (layer F.Cu) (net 1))
 (segment (start 123 37.75) (end 123 43) (width 0.25) (layer B.Cu) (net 1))
 (segment (start 116.23 49.77) (end 116.23 54) (width 0.25) (layer B.Cu) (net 1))
 (segment (start 123 43) (end 116.23 49.77) (width 0.25) (layer B.Cu) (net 1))
 (segment (start 120.25 36.5) (end 118.80048 35.05048) (width 0.25) (layer F.Cu) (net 1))
 (segment (start 118.80048 35.05048) (end 118.80048 34.25) (width 0.25) (layer F.Cu) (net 1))
 (segment (start 116.23 54) (end 116.23 52.73) (width 0.25) (layer F.Cu) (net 1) (status 10))
 (segment (start 116.23 52.73) (end 115.25 51.75) (width 0.25) (layer F.Cu) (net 1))
 (segment (start 115.25 51.75) (end 113.75 51.75) (width 0.25) (layer F.Cu) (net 1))
 (segment (start 113.75 51.75) (end 113.25 51.25) (width 0.25) (layer F.Cu) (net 1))
 (segment (start 113.25 51.25) (end 113.25 45.54928) (width 0.25) (layer F.Cu) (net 1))
 (segment (start 115.54928 44.65012) (end 115.09988 44.65012) (width 0.25) (layer F.Cu) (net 1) (status 10))
 (segment (start 114.64758 45.10242) (end 114.64758 45.54928) (width 0.25) (layer F.Cu) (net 1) (status 20))
 (segment (start 115.09988 44.65012) (end 114.64758 45.10242) (width 0.25) (layer F.Cu) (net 1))
 (segment (start 114.64758 45.54928) (end 113.25 45.54928) (width 0.25) (layer F.Cu) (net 1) (status 10))
 (segment (start 113.25 45.54928) (end 112.04928 45.54928) (width 0.25) (layer F.Cu) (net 1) (status 20))
 (segment (start 112.04928 45.54928) (end 112 45.5) (width 0.25) (layer F.Cu) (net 1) (status 30))
 (segment (start 118.80048 34.25) (end 118.80048 35.05048) (width 0.25) (layer F.Cu) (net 1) (status 10))
 (segment (start 123 37.75) (end 123 39.65) (width 0.4) (layer F.Cu) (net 1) (status 20))
 (via (at 123 37.75) (size 0.9) (layers F.Cu B.Cu) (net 1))
 (segment (start 112 42.25) (end 112 43.25) (width 0.25) (layer F.Cu) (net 3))
 (segment (start 112 43.25) (end 112.25 43.5) (width 0.25) (layer F.Cu) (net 3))
 (segment (start 116.19952 44.65012) (end 116.19952 43.94952) (width 0.25) (layer F.Cu) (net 3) (status 10))
 (segment (start 115.75 43.5) (end 112.25 43.5) (width 0.25) (layer F.Cu) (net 3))
 (segment (start 116.19952 43.94952) (end 115.75 43.5) (width 0.25) (layer F.Cu) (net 3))
 (segment (start 120.34988 45.54928) (end 122.95072 45.54928) (width 0.25) (layer F.Cu) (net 4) (status 20))
 (segment (start 122.95072 45.54928) (end 123 45.5) (width 0.25) (layer F.Cu) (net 4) (status 30))
 (segment (start 123 48) (end 123 50.5) (width 0.25) (layer F.Cu) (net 5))
 (segment (start 123.85 51.35) (end 123.85 54) (width 0.25) (layer F.Cu) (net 5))
 (segment (start 123 50.5) (end 123.85 51.35) (width 0.25) (layer F.Cu) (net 5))
 (segment (start 121 42.25) (end 121 38.75) (width 0.25) (layer B.Cu) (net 6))
 (segment (start 119.98 37.73) (end 117.5 37.73) (width 0.25) (layer B.Cu) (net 6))
 (segment (start 121 38.75) (end 119.98 37.73) (width 0.25) (layer B.Cu) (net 6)) (via (at 121 42.25) (size 0.9) (layers F.Cu B.Cu) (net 6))
 (segment (start 121 42.25) (end 121.1 42.35) (width 0.25) (layer F.Cu) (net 6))
 (segment (start 121.1 42.35) (end 123 42.35) (width 0.25) (layer F.Cu) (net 6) (status 20))
 (segment (start 118.77 54) (end 118.77 52.73) (width 0.25) (layer F.Cu) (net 7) (status 10))
 (segment (start 121 47.5) (end 120.34988 47.5) (width 0.25) (layer F.Cu) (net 7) (status 20))
 (segment (start 121.399998 47.899998) (end 121 47.5) (width 0.25) (layer F.Cu) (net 7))
 (segment (start 121.399998 51.600002) (end 121.399998 47.899998) (width 0.25) (layer F.Cu) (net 7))
 (segment (start 120.75 52.25) (end 121.399998 51.600002) (width 0.25) (layer F.Cu) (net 7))
 (segment (start 119.25 52.25) (end 120.75 52.25) (width 0.25) (layer F.Cu) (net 7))
 (segment (start 118.77 52.73) (end 119.25 52.25) (width 0.25) (layer F.Cu) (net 7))
 (segment (start 120.34988 46.84976) (end 121.09976 46.84976) (width 0.25) (layer F.Cu) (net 8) (status 10))
 (segment (start 121.31 52.69) (end 121.31 54) (width 0.25) (layer F.Cu) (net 8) (status 20))
 (segment (start 121.9 52.1) (end 121.31 52.69) (width 0.25) (layer F.Cu) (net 8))
 (segment (start 121.9 47.65) (end 121.9 52.1) (width 0.25) (layer F.Cu) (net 8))
 (segment (start 121.09976 46.84976) (end 121.9 47.65) (width 0.25) (layer F.Cu) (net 8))
 (segment (start 117.5 42.5) (end 119.25 40.75) (width 0.25) (layer F.Cu) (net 9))
 (segment (start 119.25 40.75) (end 119.25 37.5) (width 0.25) (layer F.Cu) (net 9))
 (segment (start 119.25 37.5) (end 117.5 35.75) (width 0.25) (layer F.Cu) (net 9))
 (segment (start 117.5 35.75) (end 117.5 34.25) (width 0.25) (layer F.Cu) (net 9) (status 20))
 (segment (start 117.5 44.65012) (end 117.5 42.5) (width 0.25) (layer F.Cu) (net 9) (status 10))
 (segment (start 118.15024 35.40024) (end 120 37.25) (width 0.25) (layer F.Cu) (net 11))
 (segment (start 118.15024 34.25) (end 118.15024 35.40024) (width 0.25) (layer F.Cu) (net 11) (status 10))
 (segment (start 116.84976 42.59976) (end 116.5 42.25) (width 0.25) (layer F.Cu) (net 11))
 (via (at 116.5 42.25) (size 0.9) (layers F.Cu B.Cu) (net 11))
 (segment (start 119 42.25) (end 116.5 42.25) (width 0.25) (layer B.Cu) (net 11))
 (via (at 119 42.25) (size 0.9) (layers F.Cu B.Cu) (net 11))
 (segment (start 116.84976 44.65012) (end 116.84976 42.59976) (width 0.25) (layer F.Cu) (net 11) (status 10))
 (segment (start 120 41.25) (end 119 42.25) (width 0.25) (layer F.Cu) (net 11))
 (segment (start 120 37.25) (end 120 41.25) (width 0.25) (layer F.Cu) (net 11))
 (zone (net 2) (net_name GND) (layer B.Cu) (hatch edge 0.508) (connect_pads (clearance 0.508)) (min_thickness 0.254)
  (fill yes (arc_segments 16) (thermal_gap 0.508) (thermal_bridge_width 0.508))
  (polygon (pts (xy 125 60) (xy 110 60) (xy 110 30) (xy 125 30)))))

